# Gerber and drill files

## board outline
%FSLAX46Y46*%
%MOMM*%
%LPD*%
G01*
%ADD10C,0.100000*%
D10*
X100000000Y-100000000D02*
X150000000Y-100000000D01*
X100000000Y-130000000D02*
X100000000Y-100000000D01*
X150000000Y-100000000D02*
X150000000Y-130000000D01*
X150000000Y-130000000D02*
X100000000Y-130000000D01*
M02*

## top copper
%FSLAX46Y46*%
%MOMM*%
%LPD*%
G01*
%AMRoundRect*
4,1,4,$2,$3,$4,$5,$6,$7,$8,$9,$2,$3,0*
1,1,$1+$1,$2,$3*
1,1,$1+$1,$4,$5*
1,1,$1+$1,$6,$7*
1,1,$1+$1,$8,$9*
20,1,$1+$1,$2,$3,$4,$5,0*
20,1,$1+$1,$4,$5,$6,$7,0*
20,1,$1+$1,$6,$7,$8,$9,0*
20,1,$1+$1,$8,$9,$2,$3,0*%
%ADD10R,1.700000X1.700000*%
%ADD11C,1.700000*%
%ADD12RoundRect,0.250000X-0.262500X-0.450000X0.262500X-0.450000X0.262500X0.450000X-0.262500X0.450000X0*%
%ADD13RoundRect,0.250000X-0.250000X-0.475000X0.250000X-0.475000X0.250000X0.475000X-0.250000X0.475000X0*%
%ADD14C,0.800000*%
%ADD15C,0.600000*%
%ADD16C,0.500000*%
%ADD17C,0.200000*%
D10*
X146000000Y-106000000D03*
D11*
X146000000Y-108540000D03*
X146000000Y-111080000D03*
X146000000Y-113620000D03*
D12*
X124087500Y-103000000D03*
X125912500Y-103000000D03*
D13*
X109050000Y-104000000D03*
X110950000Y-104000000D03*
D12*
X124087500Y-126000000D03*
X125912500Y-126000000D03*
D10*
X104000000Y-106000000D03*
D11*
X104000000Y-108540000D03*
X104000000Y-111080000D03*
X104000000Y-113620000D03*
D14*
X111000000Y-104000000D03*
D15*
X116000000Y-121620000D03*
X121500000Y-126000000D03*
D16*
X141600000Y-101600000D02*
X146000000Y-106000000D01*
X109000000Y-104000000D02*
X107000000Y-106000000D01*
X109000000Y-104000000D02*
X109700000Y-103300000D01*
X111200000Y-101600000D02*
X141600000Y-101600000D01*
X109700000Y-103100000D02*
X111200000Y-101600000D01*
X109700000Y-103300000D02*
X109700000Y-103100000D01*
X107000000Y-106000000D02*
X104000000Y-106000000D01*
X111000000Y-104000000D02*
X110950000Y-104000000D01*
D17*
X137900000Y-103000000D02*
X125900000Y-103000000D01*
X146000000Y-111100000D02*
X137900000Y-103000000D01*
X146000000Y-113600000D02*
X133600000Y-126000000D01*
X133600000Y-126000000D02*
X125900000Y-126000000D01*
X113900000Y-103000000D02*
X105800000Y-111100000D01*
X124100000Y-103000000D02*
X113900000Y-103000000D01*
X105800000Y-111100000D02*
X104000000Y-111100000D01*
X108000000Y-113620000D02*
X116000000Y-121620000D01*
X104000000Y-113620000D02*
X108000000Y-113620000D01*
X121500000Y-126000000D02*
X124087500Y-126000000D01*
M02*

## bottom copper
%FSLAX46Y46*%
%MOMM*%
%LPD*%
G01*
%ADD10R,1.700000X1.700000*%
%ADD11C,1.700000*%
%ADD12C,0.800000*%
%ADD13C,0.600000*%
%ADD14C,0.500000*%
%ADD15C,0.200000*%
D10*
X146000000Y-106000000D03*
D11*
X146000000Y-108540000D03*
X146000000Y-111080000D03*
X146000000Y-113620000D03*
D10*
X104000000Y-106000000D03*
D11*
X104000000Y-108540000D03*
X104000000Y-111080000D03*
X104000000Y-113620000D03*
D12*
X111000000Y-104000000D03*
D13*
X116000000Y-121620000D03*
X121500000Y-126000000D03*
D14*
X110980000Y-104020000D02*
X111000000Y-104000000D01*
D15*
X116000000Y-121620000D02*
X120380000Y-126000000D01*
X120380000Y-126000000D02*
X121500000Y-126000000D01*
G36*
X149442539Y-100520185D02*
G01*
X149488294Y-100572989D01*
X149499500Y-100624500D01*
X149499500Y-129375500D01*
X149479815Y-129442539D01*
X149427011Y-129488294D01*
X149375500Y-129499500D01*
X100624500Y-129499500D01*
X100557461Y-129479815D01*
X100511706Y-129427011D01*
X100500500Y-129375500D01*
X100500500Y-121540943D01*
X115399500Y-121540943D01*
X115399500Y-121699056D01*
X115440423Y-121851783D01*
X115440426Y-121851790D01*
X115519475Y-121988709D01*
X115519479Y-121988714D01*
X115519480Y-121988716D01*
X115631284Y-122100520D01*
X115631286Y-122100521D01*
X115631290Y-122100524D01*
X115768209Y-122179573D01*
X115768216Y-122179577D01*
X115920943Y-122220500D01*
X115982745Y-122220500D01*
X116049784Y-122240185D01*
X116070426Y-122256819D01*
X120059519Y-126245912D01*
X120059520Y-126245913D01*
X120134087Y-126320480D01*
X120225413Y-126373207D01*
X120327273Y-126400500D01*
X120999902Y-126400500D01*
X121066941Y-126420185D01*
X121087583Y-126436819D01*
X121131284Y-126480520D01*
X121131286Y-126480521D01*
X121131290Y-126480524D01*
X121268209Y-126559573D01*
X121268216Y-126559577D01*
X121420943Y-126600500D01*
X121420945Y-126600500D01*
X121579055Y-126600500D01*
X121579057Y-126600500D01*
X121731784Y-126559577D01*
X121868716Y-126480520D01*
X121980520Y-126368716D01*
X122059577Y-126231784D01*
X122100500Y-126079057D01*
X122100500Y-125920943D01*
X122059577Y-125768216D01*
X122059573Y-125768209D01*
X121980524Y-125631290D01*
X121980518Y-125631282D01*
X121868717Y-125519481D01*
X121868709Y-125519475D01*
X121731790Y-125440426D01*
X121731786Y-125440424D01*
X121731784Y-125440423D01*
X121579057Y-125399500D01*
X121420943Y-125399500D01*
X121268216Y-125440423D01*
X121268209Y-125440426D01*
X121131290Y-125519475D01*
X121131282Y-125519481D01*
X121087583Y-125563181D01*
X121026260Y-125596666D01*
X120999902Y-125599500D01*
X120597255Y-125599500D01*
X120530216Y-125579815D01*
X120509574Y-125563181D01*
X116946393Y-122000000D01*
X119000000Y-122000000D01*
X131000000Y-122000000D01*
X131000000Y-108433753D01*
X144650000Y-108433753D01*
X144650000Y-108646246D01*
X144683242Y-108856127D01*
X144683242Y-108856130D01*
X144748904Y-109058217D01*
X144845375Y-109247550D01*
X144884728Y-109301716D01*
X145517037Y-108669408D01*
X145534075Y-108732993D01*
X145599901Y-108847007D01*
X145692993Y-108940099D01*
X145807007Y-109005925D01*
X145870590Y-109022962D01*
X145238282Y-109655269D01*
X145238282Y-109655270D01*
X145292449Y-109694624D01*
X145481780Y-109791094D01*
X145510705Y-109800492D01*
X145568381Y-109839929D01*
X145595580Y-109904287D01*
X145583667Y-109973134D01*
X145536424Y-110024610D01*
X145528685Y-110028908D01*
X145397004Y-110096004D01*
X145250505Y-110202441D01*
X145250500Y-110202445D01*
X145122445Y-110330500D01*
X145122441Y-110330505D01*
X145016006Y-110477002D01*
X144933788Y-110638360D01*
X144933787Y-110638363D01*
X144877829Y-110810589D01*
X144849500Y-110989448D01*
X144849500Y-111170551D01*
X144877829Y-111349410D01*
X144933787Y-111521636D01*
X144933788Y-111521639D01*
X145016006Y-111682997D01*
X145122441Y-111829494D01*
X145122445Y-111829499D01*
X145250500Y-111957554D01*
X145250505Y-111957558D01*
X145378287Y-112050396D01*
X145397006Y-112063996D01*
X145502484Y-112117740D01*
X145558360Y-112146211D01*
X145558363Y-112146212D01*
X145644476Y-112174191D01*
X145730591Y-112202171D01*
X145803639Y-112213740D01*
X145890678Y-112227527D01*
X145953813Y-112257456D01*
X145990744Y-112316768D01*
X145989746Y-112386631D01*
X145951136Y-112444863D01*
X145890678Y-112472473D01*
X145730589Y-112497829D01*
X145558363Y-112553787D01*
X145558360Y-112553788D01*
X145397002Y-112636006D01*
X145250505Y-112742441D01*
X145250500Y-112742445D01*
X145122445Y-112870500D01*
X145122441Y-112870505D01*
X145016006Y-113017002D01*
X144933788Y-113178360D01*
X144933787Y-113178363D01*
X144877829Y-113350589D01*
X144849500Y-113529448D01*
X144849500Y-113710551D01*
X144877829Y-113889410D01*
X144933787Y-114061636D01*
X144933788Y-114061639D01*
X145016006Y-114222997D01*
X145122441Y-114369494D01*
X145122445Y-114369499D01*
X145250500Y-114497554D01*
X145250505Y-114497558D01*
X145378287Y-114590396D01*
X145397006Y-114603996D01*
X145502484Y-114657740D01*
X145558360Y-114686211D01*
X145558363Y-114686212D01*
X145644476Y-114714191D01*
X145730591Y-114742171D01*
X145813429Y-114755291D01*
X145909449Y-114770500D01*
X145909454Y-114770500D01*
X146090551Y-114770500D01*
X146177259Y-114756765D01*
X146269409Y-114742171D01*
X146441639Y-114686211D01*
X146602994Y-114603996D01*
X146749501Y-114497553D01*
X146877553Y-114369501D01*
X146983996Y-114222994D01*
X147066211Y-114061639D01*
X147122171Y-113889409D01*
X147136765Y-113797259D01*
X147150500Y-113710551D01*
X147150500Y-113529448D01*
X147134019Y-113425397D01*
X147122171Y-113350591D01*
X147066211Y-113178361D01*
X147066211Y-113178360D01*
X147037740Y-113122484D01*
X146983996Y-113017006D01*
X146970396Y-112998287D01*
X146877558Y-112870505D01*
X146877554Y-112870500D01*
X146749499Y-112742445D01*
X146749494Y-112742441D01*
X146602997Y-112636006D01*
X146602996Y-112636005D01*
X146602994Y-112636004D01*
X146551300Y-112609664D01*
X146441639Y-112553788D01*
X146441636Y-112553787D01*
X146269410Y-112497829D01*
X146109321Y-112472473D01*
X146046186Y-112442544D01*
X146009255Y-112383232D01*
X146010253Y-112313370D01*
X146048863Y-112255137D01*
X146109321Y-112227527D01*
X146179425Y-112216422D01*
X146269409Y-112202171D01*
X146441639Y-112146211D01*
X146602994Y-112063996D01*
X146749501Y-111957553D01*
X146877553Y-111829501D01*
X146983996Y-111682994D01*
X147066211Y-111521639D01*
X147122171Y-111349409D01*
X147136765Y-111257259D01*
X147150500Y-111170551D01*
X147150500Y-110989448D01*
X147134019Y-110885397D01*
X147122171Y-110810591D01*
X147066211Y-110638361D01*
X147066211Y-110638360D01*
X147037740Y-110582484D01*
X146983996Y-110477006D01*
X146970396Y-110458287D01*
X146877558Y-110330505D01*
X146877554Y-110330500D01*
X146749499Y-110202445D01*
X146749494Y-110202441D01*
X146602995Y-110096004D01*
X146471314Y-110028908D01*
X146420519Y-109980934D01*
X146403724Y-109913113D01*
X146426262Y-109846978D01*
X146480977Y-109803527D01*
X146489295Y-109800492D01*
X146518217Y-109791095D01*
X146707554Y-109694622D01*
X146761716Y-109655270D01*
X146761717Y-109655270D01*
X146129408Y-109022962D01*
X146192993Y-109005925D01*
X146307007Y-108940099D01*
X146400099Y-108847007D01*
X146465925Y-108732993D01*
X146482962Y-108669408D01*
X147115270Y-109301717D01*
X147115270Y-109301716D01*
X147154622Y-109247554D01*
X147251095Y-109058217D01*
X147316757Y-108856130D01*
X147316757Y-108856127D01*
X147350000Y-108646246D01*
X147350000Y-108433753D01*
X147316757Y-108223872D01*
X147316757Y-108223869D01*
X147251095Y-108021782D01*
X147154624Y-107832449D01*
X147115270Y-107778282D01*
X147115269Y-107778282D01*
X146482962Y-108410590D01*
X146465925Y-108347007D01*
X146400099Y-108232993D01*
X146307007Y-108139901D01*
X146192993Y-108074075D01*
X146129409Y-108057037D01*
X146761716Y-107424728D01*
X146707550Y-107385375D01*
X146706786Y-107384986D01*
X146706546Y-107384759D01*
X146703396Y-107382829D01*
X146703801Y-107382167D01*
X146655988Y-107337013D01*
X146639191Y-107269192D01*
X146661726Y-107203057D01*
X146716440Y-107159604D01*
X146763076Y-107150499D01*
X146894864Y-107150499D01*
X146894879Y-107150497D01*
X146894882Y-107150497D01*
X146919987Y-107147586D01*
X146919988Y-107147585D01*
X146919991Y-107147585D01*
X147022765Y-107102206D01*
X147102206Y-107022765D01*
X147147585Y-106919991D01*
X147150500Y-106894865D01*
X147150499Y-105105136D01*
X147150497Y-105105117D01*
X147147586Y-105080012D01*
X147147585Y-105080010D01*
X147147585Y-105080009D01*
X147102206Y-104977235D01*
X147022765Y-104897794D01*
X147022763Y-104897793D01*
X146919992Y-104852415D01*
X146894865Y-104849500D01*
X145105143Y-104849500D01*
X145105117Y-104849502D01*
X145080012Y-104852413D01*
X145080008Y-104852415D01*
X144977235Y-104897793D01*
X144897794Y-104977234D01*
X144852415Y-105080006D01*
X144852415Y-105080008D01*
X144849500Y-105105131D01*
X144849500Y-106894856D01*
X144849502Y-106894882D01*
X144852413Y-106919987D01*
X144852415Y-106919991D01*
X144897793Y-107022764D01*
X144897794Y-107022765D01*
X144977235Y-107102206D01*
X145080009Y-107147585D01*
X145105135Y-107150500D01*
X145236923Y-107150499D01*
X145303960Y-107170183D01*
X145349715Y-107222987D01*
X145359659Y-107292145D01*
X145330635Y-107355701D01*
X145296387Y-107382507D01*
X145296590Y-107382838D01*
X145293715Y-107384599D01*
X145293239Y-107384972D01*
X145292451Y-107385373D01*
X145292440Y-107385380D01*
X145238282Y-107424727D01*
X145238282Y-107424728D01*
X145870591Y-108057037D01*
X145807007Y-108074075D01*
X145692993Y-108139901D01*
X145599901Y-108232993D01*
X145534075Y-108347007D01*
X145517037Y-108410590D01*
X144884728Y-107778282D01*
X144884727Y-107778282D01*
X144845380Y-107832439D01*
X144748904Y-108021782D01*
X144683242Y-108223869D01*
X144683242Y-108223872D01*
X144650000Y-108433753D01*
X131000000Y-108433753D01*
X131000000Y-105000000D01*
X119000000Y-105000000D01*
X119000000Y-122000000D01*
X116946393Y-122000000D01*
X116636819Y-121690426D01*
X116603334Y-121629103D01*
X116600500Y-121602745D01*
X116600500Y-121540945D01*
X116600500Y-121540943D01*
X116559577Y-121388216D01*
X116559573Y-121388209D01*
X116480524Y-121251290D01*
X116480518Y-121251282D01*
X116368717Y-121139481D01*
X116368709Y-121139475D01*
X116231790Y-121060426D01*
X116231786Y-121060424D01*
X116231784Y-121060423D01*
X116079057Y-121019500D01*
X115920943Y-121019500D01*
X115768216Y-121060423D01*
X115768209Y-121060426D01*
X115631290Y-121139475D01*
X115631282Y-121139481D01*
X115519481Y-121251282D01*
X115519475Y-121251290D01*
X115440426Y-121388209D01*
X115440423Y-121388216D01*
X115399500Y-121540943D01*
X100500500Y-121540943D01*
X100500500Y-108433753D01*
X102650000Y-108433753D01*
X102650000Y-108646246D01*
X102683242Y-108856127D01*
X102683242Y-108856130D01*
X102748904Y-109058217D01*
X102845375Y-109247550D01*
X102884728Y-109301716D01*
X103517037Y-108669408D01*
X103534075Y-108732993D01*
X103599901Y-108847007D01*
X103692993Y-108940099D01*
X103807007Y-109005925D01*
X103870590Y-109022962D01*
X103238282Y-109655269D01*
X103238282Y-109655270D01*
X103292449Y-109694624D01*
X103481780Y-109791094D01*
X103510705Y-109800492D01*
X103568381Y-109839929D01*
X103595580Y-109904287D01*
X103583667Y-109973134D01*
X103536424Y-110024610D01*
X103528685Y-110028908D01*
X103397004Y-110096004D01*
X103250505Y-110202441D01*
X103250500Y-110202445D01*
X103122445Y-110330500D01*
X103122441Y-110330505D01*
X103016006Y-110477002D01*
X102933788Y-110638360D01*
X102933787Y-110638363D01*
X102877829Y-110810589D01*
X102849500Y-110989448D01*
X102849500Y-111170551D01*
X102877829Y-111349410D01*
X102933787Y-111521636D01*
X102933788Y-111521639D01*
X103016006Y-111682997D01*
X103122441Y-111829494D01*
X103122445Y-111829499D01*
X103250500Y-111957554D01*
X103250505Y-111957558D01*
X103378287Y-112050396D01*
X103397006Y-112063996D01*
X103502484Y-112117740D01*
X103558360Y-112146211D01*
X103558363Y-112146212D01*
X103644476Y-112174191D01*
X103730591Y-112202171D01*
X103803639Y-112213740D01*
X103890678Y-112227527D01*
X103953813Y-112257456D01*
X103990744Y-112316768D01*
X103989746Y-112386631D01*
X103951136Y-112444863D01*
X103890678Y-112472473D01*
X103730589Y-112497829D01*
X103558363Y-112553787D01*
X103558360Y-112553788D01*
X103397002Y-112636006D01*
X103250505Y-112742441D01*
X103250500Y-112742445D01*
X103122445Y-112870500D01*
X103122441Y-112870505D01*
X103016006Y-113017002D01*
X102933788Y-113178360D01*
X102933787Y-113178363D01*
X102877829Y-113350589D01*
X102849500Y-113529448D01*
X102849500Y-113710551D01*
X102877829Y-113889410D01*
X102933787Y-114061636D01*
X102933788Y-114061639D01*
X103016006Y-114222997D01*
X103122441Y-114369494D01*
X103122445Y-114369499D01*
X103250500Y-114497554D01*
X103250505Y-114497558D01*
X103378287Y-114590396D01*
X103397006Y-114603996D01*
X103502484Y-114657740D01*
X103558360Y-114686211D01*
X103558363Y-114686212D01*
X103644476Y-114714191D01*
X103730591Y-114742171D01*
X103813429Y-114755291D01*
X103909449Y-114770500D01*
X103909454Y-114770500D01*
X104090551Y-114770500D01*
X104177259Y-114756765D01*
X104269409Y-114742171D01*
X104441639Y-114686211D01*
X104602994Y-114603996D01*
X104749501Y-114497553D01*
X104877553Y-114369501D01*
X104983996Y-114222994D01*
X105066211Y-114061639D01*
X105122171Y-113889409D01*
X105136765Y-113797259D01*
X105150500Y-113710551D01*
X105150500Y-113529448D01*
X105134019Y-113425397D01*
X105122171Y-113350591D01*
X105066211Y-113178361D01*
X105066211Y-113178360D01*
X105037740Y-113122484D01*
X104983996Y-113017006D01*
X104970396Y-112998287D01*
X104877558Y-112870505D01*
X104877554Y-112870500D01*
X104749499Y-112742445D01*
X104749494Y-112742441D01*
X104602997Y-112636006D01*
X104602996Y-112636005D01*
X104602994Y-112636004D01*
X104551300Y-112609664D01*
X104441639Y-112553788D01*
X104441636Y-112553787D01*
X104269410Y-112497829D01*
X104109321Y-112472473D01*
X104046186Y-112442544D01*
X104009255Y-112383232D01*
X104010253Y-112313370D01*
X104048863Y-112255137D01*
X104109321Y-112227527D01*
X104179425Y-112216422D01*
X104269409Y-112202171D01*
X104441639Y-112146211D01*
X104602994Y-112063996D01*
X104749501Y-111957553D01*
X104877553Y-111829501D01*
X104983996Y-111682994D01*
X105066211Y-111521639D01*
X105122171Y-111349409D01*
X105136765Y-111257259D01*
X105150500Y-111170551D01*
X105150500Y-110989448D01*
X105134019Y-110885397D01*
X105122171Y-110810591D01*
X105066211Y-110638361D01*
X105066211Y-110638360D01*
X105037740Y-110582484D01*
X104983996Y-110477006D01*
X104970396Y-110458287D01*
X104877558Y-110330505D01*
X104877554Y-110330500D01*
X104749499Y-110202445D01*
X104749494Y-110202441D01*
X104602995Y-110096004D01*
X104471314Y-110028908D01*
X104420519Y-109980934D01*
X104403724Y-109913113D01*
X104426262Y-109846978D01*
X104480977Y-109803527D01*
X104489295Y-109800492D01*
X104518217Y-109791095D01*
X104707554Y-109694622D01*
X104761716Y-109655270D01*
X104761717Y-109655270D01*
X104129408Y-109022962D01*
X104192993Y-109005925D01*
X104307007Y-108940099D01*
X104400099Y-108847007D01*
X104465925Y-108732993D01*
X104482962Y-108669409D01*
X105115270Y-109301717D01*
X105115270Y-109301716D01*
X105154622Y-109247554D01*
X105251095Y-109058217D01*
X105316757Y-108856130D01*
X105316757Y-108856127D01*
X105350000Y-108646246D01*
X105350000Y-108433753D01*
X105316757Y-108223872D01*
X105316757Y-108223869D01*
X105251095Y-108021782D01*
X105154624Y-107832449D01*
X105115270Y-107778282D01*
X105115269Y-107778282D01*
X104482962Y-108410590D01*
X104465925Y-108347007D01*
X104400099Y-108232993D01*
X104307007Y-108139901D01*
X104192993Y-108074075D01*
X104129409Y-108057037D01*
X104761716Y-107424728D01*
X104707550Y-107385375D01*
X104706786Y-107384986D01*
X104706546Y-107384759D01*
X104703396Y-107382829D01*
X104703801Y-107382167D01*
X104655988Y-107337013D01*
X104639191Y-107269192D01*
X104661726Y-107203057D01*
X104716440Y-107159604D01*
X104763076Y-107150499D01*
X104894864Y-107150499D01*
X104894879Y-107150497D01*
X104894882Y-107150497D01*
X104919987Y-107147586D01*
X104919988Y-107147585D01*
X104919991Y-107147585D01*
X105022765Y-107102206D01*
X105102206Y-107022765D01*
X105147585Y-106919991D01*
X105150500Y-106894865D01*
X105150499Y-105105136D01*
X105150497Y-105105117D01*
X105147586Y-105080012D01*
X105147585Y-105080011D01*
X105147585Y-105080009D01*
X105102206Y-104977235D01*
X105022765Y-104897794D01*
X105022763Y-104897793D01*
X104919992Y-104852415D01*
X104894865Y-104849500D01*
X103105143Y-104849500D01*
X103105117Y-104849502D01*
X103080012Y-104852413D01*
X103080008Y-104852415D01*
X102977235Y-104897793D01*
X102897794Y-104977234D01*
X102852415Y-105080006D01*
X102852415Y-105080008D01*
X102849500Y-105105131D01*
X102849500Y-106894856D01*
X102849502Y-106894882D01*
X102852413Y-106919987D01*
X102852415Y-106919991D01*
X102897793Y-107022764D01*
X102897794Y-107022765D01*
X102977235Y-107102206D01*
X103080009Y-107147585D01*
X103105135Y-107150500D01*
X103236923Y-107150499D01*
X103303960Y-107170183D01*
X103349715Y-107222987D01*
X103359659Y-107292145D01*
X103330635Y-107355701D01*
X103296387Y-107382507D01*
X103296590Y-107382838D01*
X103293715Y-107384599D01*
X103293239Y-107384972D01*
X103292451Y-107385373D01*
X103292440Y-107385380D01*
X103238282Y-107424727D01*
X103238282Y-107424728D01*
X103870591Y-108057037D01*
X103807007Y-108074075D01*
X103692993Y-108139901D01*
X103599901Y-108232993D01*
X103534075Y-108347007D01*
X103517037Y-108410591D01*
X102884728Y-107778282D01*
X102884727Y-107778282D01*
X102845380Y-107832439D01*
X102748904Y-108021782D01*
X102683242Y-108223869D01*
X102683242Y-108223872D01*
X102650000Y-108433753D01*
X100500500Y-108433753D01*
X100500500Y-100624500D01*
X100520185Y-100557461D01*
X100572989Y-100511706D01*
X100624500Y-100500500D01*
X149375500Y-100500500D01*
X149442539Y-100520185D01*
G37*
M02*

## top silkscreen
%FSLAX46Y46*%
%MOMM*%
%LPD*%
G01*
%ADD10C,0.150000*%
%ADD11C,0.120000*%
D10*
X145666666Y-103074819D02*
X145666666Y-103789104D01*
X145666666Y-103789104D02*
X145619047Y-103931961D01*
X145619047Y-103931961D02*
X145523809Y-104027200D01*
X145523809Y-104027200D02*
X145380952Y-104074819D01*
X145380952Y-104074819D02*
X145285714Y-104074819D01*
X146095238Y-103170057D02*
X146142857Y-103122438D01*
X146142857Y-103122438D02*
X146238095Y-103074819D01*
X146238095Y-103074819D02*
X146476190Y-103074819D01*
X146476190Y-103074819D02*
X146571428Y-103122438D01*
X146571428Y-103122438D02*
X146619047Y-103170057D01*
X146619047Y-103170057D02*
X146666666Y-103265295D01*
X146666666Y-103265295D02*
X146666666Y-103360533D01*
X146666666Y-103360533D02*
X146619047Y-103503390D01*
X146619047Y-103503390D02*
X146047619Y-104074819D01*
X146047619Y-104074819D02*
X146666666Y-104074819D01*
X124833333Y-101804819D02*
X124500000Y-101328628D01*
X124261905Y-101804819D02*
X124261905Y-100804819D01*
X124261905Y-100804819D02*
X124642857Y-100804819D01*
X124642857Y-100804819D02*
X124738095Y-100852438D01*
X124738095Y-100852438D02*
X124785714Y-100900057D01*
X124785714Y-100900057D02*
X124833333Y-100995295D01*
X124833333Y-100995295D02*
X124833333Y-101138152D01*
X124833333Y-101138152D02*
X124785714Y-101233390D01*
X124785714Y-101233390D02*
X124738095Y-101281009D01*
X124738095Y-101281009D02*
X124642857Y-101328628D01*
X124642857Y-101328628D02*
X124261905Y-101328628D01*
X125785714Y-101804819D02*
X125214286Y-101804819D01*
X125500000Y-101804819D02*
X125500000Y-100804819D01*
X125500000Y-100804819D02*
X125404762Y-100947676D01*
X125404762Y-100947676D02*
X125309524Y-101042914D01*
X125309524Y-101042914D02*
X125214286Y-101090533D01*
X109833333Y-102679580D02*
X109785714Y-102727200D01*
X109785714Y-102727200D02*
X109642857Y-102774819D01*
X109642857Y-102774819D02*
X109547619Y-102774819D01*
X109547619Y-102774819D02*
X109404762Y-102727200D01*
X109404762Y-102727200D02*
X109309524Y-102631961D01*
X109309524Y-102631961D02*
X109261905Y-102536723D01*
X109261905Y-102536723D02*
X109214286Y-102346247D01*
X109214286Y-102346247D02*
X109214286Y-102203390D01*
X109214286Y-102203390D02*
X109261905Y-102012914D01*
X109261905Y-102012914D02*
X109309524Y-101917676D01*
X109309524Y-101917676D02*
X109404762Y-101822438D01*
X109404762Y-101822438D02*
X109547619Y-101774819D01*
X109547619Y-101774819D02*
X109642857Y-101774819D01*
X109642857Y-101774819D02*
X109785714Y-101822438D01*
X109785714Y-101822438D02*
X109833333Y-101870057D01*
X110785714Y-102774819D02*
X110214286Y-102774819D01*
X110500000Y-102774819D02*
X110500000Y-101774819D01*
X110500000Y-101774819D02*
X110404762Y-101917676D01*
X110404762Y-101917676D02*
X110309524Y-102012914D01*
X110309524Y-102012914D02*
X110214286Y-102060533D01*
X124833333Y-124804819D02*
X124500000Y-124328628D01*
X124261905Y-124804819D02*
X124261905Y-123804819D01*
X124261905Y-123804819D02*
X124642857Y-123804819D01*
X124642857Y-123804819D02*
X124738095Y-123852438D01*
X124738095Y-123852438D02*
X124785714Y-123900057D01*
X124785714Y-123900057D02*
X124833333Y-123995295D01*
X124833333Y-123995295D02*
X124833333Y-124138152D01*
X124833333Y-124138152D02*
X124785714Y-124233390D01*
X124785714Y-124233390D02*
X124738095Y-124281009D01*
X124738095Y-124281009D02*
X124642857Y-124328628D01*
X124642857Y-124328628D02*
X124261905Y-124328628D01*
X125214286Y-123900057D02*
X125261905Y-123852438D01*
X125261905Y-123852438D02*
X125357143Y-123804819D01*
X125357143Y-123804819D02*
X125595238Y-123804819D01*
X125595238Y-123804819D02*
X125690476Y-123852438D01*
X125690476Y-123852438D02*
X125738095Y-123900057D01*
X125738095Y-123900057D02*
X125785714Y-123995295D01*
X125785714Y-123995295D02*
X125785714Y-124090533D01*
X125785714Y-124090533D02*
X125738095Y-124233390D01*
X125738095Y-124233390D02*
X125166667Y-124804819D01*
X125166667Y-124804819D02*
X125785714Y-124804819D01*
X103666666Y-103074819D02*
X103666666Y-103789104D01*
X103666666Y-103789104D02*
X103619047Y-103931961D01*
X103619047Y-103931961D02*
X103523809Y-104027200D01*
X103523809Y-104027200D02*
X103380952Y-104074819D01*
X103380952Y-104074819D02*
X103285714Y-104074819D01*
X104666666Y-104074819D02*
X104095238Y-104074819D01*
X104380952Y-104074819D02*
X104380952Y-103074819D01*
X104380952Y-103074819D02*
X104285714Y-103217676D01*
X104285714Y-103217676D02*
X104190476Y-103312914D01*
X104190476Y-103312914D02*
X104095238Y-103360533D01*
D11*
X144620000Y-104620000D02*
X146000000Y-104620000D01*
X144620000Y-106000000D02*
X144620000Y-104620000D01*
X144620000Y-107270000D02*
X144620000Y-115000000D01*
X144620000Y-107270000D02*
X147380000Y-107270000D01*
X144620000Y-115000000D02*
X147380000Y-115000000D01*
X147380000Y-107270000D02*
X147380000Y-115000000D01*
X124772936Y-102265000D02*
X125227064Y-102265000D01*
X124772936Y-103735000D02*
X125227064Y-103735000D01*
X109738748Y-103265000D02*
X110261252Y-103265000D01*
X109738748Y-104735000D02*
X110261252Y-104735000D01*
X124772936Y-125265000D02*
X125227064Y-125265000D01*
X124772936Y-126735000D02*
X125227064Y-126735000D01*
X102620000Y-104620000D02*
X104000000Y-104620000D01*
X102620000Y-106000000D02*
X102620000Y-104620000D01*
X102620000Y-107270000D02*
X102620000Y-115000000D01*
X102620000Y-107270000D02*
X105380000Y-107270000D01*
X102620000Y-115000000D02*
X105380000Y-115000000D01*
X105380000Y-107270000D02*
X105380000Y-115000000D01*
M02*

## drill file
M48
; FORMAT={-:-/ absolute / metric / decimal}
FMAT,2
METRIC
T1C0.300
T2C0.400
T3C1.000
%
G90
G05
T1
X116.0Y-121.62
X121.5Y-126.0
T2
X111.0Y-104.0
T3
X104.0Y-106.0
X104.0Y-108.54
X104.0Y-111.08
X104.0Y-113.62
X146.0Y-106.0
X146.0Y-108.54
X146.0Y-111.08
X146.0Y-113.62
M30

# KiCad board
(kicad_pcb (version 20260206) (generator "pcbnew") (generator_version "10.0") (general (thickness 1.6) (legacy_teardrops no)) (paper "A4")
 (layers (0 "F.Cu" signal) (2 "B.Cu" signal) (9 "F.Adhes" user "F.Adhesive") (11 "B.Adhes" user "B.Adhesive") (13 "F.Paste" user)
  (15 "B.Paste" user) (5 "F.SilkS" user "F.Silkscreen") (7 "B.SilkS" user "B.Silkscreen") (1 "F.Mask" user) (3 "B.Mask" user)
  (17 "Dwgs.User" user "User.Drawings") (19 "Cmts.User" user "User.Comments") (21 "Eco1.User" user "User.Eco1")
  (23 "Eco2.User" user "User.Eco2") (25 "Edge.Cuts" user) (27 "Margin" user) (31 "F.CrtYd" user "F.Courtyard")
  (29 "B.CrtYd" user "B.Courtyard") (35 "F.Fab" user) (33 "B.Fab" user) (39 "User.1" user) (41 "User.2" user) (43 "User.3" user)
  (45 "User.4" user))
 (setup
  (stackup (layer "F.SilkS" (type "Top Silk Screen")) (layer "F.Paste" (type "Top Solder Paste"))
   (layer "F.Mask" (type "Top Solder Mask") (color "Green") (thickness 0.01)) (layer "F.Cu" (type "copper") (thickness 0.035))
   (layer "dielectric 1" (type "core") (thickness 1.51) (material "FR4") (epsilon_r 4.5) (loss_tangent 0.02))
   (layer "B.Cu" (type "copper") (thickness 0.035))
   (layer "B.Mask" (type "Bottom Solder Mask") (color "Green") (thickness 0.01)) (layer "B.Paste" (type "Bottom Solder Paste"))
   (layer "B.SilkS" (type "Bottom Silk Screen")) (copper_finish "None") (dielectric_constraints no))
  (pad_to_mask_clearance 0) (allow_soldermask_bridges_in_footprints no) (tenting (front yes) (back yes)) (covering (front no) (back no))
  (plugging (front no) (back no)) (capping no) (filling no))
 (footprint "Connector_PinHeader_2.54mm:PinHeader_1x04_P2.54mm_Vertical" (layer "F.Cu") (at 146 106)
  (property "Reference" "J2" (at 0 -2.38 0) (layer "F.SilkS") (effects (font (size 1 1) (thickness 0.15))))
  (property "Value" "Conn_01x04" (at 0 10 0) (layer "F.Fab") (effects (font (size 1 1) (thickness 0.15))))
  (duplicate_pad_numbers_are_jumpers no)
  (fp_line (start -1.38 -1.38) (end 0 -1.38) (stroke (width 0.12) (type solid)) (layer "F.SilkS"))
  (fp_line (start -1.38 0) (end -1.38 -1.38) (stroke (width 0.12) (type solid)) (layer "F.SilkS"))
  (fp_line (start -1.38 1.27) (end -1.38 9) (stroke (width 0.12) (type solid)) (layer "F.SilkS"))
  (fp_line (start -1.38 1.27) (end 1.38 1.27) (stroke (width 0.12) (type solid)) (layer "F.SilkS"))
  (fp_line (start -1.38 9) (end 1.38 9) (stroke (width 0.12) (type solid)) (layer "F.SilkS"))
  (fp_line (start 1.38 1.27) (end 1.38 9) (stroke (width 0.12) (type solid)) (layer "F.SilkS"))
  (pad "1" thru_hole rect (at 0 0) (size 1.7 1.7) (drill 1) (layers "*.Cu" "*.Mask") (remove_unused_layers no) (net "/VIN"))
  (pad "2" thru_hole circle (at 0 2.54) (size 1.7 1.7) (drill 1) (layers "*.Cu" "*.Mask") (remove_unused_layers no) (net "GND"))
  (pad "3" thru_hole circle (at 0 5.08) (size 1.7 1.7) (drill 1) (layers "*.Cu" "*.Mask") (remove_unused_layers no) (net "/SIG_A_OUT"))
  (pad "4" thru_hole circle (at 0 7.62) (size 1.7 1.7) (drill 1) (layers "*.Cu" "*.Mask") (remove_unused_layers no) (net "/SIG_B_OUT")))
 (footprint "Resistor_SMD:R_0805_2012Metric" (layer "F.Cu") (at 125 103)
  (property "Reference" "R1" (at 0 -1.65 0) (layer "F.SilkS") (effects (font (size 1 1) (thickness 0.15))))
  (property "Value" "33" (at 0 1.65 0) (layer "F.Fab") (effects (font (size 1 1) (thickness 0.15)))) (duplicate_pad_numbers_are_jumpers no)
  (fp_line (start -0.227064 -0.735) (end 0.227064 -0.735) (stroke (width 0.12) (type solid)) (layer "F.SilkS"))
  (fp_line (start -0.227064 0.735) (end 0.227064 0.735) (stroke (width 0.12) (type solid)) (layer "F.SilkS"))
  (pad "1" smd roundrect (at -0.9125 0) (size 1.025 1.4) (layers "F.Cu" "F.Mask" "F.Paste") (roundrect_rratio 0.243902) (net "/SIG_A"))
  (pad "2" smd roundrect (at 0.9125 0) (size 1.025 1.4) (layers "F.Cu" "F.Mask" "F.Paste") (roundrect_rratio 0.243902) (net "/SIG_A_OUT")))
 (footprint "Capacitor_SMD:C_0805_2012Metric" (layer "F.Cu") (at 110 104)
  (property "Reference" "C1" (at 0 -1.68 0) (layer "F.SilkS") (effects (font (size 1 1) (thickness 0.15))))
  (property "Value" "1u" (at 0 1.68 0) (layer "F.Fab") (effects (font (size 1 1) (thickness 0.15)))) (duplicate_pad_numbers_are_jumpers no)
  (fp_line (start -0.261252 -0.735) (end 0.261252 -0.735) (stroke (width 0.12) (type solid)) (layer "F.SilkS"))
  (fp_line (start -0.261252 0.735) (end 0.261252 0.735) (stroke (width 0.12) (type solid)) (layer "F.SilkS"))
  (pad "1" smd roundrect (at -0.95 0) (size 1 1.45) (layers "F.Cu" "F.Mask" "F.Paste") (roundrect_rratio 0.25) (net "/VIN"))
  (pad "2" smd roundrect (at 0.95 0) (size 1 1.45) (layers "F.Cu" "F.Mask" "F.Paste") (roundrect_rratio 0.25) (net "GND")))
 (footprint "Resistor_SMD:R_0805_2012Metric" (layer "F.Cu") (at 125 126)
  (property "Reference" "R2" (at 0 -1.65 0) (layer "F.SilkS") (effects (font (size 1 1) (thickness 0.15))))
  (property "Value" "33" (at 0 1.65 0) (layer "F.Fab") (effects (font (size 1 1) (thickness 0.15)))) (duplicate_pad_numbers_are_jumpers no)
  (fp_line (start -0.227064 -0.735) (end 0.227064 -0.735) (stroke (width 0.12) (type solid)) (layer "F.SilkS"))
  (fp_line (start -0.227064 0.735) (end 0.227064 0.735) (stroke (width 0.12) (type solid)) (layer "F.SilkS"))
  (pad "1" smd roundrect (at -0.9125 0) (size 1.025 1.4) (layers "F.Cu" "F.Mask" "F.Paste") (roundrect_rratio 0.243902) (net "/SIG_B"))
  (pad "2" smd roundrect (at 0.9125 0) (size 1.025 1.4) (layers "F.Cu" "F.Mask" "F.Paste") (roundrect_rratio 0.243902) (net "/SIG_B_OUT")))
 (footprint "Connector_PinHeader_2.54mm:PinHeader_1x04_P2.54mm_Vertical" (layer "F.Cu") (at 104 106)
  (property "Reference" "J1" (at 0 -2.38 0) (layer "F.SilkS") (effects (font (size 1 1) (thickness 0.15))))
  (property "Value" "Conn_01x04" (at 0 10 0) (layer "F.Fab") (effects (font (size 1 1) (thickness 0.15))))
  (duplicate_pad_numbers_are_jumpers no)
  (fp_line (start -1.38 -1.38) (end 0 -1.38) (stroke (width 0.12) (type solid)) (layer "F.SilkS"))
  (fp_line (start -1.38 0) (end -1.38 -1.38) (stroke (width 0.12) (type solid)) (layer "F.SilkS"))
  (fp_line (start -1.38 1.27) (end -1.38 9) (stroke (width 0.12) (type solid)) (layer "F.SilkS"))
  (fp_line (start -1.38 1.27) (end 1.38 1.27) (stroke (width 0.12) (type solid)) (layer "F.SilkS"))
  (fp_line (start -1.38 9) (end 1.38 9) (stroke (width 0.12) (type solid)) (layer "F.SilkS"))
  (fp_line (start 1.38 1.27) (end 1.38 9) (stroke (width 0.12) (type solid)) (layer "F.SilkS"))
  (pad "1" thru_hole rect (at 0 0) (size 1.7 1.7) (drill 1) (layers "*.Cu" "*.Mask") (remove_unused_layers no) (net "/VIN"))
  (pad "2" thru_hole circle (at 0 2.54) (size 1.7 1.7) (drill 1) (layers "*.Cu" "*.Mask") (remove_unused_layers no) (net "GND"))
  (pad "3" thru_hole circle (at 0 5.08) (size 1.7 1.7) (drill 1) (layers "*.Cu" "*.Mask") (remove_unused_layers no) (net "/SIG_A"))
  (pad "4" thru_hole circle (at 0 7.62) (size 1.7 1.7) (drill 1) (layers "*.Cu" "*.Mask") (remove_unused_layers no) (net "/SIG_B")))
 (gr_line (start 100 100) (end 150 100) (stroke (width 0.1) (type default)) (layer "Edge.Cuts"))
 (gr_line (start 100 130) (end 100 100) (stroke (width 0.1) (type default)) (layer "Edge.Cuts"))
 (gr_line (start 150 100) (end 150 130) (stroke (width 0.1) (type default)) (layer "Edge.Cuts"))
 (gr_line (start 150 130) (end 100 130) (stroke (width 0.1) (type default)) (layer "Edge.Cuts"))
 (segment (start 141.6 101.6) (end 146 106) (width 0.5) (layer "F.Cu") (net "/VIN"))
 (segment (start 109 104) (end 107 106) (width 0.5) (layer "F.Cu") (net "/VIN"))
 (segment (start 109 104) (end 109.7 103.3) (width 0.5) (layer "F.Cu") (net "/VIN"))
 (segment (start 111.2 101.6) (end 141.6 101.6) (width 0.5) (layer "F.Cu") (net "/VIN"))
 (segment (start 109.7 103.1) (end 111.2 101.6) (width 0.5) (layer "F.Cu") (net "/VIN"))
 (segment (start 109.7 103.3) (end 109.7 103.1) (width 0.5) (layer "F.Cu") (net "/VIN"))
 (segment (start 107 106) (end 104 106) (width 0.5) (layer "F.Cu") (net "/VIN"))
 (segment (start 111 104) (end 110.95 104) (width 0.5) (layer "F.Cu") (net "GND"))
 (via (at 111 104) (size 0.8) (drill 0.4) (layers "F.Cu" "B.Cu") (capping yes) (filling yes) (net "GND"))
 (segment (start 110.98 104.02) (end 111 104) (width 0.5) (layer "B.Cu") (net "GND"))
 (segment (start 137.9 103) (end 125.9 103) (width 0.2) (layer "F.Cu") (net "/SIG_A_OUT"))
 (segment (start 146 111.1) (end 137.9 103) (width 0.2) (layer "F.Cu") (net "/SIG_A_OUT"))
 (segment (start 146 113.6) (end 133.6 126) (width 0.2) (layer "F.Cu") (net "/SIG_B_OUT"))
 (segment (start 133.6 126) (end 125.9 126) (width 0.2) (layer "F.Cu") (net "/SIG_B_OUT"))
 (segment (start 113.9 103) (end 105.8 111.1) (width 0.2) (layer "F.Cu") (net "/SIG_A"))
 (segment (start 124.1 103) (end 113.9 103) (width 0.2) (layer "F.Cu") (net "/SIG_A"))
 (segment (start 105.8 111.1) (end 104 111.1) (width 0.2) (layer "F.Cu") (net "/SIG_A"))
 (segment (start 108 113.62) (end 116 121.62) (width 0.2) (locked yes) (layer "F.Cu") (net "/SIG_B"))
 (segment (start 104 113.62) (end 108 113.62) (width 0.2) (locked yes) (layer "F.Cu") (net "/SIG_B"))
 (segment (start 121.5 126) (end 124.0875 126) (width 0.2) (locked yes) (layer "F.Cu") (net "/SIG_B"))
 (via (at 116 121.62) (size 0.6) (drill 0.3) (layers "F.Cu" "B.Cu") (locked yes) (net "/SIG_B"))
 (via (at 121.5 126) (size 0.6) (drill 0.3) (layers "F.Cu" "B.Cu") (locked yes) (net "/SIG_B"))
 (segment (start 116 121.62) (end 120.38 126) (width 0.2) (locked yes) (layer "B.Cu") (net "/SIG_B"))
 (segment (start 120.38 126) (end 121.5 126) (width 0.2) (locked yes) (layer "B.Cu") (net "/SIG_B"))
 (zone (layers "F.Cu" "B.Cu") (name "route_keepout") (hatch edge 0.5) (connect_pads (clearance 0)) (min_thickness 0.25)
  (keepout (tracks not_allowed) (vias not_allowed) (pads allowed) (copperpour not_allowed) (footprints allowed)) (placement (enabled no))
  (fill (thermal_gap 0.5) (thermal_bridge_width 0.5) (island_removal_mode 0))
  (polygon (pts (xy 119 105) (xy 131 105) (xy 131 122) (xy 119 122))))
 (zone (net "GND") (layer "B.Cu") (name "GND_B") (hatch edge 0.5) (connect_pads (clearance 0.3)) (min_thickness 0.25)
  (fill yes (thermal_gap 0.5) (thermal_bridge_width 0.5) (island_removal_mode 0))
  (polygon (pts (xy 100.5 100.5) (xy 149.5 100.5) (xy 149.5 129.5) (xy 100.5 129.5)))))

